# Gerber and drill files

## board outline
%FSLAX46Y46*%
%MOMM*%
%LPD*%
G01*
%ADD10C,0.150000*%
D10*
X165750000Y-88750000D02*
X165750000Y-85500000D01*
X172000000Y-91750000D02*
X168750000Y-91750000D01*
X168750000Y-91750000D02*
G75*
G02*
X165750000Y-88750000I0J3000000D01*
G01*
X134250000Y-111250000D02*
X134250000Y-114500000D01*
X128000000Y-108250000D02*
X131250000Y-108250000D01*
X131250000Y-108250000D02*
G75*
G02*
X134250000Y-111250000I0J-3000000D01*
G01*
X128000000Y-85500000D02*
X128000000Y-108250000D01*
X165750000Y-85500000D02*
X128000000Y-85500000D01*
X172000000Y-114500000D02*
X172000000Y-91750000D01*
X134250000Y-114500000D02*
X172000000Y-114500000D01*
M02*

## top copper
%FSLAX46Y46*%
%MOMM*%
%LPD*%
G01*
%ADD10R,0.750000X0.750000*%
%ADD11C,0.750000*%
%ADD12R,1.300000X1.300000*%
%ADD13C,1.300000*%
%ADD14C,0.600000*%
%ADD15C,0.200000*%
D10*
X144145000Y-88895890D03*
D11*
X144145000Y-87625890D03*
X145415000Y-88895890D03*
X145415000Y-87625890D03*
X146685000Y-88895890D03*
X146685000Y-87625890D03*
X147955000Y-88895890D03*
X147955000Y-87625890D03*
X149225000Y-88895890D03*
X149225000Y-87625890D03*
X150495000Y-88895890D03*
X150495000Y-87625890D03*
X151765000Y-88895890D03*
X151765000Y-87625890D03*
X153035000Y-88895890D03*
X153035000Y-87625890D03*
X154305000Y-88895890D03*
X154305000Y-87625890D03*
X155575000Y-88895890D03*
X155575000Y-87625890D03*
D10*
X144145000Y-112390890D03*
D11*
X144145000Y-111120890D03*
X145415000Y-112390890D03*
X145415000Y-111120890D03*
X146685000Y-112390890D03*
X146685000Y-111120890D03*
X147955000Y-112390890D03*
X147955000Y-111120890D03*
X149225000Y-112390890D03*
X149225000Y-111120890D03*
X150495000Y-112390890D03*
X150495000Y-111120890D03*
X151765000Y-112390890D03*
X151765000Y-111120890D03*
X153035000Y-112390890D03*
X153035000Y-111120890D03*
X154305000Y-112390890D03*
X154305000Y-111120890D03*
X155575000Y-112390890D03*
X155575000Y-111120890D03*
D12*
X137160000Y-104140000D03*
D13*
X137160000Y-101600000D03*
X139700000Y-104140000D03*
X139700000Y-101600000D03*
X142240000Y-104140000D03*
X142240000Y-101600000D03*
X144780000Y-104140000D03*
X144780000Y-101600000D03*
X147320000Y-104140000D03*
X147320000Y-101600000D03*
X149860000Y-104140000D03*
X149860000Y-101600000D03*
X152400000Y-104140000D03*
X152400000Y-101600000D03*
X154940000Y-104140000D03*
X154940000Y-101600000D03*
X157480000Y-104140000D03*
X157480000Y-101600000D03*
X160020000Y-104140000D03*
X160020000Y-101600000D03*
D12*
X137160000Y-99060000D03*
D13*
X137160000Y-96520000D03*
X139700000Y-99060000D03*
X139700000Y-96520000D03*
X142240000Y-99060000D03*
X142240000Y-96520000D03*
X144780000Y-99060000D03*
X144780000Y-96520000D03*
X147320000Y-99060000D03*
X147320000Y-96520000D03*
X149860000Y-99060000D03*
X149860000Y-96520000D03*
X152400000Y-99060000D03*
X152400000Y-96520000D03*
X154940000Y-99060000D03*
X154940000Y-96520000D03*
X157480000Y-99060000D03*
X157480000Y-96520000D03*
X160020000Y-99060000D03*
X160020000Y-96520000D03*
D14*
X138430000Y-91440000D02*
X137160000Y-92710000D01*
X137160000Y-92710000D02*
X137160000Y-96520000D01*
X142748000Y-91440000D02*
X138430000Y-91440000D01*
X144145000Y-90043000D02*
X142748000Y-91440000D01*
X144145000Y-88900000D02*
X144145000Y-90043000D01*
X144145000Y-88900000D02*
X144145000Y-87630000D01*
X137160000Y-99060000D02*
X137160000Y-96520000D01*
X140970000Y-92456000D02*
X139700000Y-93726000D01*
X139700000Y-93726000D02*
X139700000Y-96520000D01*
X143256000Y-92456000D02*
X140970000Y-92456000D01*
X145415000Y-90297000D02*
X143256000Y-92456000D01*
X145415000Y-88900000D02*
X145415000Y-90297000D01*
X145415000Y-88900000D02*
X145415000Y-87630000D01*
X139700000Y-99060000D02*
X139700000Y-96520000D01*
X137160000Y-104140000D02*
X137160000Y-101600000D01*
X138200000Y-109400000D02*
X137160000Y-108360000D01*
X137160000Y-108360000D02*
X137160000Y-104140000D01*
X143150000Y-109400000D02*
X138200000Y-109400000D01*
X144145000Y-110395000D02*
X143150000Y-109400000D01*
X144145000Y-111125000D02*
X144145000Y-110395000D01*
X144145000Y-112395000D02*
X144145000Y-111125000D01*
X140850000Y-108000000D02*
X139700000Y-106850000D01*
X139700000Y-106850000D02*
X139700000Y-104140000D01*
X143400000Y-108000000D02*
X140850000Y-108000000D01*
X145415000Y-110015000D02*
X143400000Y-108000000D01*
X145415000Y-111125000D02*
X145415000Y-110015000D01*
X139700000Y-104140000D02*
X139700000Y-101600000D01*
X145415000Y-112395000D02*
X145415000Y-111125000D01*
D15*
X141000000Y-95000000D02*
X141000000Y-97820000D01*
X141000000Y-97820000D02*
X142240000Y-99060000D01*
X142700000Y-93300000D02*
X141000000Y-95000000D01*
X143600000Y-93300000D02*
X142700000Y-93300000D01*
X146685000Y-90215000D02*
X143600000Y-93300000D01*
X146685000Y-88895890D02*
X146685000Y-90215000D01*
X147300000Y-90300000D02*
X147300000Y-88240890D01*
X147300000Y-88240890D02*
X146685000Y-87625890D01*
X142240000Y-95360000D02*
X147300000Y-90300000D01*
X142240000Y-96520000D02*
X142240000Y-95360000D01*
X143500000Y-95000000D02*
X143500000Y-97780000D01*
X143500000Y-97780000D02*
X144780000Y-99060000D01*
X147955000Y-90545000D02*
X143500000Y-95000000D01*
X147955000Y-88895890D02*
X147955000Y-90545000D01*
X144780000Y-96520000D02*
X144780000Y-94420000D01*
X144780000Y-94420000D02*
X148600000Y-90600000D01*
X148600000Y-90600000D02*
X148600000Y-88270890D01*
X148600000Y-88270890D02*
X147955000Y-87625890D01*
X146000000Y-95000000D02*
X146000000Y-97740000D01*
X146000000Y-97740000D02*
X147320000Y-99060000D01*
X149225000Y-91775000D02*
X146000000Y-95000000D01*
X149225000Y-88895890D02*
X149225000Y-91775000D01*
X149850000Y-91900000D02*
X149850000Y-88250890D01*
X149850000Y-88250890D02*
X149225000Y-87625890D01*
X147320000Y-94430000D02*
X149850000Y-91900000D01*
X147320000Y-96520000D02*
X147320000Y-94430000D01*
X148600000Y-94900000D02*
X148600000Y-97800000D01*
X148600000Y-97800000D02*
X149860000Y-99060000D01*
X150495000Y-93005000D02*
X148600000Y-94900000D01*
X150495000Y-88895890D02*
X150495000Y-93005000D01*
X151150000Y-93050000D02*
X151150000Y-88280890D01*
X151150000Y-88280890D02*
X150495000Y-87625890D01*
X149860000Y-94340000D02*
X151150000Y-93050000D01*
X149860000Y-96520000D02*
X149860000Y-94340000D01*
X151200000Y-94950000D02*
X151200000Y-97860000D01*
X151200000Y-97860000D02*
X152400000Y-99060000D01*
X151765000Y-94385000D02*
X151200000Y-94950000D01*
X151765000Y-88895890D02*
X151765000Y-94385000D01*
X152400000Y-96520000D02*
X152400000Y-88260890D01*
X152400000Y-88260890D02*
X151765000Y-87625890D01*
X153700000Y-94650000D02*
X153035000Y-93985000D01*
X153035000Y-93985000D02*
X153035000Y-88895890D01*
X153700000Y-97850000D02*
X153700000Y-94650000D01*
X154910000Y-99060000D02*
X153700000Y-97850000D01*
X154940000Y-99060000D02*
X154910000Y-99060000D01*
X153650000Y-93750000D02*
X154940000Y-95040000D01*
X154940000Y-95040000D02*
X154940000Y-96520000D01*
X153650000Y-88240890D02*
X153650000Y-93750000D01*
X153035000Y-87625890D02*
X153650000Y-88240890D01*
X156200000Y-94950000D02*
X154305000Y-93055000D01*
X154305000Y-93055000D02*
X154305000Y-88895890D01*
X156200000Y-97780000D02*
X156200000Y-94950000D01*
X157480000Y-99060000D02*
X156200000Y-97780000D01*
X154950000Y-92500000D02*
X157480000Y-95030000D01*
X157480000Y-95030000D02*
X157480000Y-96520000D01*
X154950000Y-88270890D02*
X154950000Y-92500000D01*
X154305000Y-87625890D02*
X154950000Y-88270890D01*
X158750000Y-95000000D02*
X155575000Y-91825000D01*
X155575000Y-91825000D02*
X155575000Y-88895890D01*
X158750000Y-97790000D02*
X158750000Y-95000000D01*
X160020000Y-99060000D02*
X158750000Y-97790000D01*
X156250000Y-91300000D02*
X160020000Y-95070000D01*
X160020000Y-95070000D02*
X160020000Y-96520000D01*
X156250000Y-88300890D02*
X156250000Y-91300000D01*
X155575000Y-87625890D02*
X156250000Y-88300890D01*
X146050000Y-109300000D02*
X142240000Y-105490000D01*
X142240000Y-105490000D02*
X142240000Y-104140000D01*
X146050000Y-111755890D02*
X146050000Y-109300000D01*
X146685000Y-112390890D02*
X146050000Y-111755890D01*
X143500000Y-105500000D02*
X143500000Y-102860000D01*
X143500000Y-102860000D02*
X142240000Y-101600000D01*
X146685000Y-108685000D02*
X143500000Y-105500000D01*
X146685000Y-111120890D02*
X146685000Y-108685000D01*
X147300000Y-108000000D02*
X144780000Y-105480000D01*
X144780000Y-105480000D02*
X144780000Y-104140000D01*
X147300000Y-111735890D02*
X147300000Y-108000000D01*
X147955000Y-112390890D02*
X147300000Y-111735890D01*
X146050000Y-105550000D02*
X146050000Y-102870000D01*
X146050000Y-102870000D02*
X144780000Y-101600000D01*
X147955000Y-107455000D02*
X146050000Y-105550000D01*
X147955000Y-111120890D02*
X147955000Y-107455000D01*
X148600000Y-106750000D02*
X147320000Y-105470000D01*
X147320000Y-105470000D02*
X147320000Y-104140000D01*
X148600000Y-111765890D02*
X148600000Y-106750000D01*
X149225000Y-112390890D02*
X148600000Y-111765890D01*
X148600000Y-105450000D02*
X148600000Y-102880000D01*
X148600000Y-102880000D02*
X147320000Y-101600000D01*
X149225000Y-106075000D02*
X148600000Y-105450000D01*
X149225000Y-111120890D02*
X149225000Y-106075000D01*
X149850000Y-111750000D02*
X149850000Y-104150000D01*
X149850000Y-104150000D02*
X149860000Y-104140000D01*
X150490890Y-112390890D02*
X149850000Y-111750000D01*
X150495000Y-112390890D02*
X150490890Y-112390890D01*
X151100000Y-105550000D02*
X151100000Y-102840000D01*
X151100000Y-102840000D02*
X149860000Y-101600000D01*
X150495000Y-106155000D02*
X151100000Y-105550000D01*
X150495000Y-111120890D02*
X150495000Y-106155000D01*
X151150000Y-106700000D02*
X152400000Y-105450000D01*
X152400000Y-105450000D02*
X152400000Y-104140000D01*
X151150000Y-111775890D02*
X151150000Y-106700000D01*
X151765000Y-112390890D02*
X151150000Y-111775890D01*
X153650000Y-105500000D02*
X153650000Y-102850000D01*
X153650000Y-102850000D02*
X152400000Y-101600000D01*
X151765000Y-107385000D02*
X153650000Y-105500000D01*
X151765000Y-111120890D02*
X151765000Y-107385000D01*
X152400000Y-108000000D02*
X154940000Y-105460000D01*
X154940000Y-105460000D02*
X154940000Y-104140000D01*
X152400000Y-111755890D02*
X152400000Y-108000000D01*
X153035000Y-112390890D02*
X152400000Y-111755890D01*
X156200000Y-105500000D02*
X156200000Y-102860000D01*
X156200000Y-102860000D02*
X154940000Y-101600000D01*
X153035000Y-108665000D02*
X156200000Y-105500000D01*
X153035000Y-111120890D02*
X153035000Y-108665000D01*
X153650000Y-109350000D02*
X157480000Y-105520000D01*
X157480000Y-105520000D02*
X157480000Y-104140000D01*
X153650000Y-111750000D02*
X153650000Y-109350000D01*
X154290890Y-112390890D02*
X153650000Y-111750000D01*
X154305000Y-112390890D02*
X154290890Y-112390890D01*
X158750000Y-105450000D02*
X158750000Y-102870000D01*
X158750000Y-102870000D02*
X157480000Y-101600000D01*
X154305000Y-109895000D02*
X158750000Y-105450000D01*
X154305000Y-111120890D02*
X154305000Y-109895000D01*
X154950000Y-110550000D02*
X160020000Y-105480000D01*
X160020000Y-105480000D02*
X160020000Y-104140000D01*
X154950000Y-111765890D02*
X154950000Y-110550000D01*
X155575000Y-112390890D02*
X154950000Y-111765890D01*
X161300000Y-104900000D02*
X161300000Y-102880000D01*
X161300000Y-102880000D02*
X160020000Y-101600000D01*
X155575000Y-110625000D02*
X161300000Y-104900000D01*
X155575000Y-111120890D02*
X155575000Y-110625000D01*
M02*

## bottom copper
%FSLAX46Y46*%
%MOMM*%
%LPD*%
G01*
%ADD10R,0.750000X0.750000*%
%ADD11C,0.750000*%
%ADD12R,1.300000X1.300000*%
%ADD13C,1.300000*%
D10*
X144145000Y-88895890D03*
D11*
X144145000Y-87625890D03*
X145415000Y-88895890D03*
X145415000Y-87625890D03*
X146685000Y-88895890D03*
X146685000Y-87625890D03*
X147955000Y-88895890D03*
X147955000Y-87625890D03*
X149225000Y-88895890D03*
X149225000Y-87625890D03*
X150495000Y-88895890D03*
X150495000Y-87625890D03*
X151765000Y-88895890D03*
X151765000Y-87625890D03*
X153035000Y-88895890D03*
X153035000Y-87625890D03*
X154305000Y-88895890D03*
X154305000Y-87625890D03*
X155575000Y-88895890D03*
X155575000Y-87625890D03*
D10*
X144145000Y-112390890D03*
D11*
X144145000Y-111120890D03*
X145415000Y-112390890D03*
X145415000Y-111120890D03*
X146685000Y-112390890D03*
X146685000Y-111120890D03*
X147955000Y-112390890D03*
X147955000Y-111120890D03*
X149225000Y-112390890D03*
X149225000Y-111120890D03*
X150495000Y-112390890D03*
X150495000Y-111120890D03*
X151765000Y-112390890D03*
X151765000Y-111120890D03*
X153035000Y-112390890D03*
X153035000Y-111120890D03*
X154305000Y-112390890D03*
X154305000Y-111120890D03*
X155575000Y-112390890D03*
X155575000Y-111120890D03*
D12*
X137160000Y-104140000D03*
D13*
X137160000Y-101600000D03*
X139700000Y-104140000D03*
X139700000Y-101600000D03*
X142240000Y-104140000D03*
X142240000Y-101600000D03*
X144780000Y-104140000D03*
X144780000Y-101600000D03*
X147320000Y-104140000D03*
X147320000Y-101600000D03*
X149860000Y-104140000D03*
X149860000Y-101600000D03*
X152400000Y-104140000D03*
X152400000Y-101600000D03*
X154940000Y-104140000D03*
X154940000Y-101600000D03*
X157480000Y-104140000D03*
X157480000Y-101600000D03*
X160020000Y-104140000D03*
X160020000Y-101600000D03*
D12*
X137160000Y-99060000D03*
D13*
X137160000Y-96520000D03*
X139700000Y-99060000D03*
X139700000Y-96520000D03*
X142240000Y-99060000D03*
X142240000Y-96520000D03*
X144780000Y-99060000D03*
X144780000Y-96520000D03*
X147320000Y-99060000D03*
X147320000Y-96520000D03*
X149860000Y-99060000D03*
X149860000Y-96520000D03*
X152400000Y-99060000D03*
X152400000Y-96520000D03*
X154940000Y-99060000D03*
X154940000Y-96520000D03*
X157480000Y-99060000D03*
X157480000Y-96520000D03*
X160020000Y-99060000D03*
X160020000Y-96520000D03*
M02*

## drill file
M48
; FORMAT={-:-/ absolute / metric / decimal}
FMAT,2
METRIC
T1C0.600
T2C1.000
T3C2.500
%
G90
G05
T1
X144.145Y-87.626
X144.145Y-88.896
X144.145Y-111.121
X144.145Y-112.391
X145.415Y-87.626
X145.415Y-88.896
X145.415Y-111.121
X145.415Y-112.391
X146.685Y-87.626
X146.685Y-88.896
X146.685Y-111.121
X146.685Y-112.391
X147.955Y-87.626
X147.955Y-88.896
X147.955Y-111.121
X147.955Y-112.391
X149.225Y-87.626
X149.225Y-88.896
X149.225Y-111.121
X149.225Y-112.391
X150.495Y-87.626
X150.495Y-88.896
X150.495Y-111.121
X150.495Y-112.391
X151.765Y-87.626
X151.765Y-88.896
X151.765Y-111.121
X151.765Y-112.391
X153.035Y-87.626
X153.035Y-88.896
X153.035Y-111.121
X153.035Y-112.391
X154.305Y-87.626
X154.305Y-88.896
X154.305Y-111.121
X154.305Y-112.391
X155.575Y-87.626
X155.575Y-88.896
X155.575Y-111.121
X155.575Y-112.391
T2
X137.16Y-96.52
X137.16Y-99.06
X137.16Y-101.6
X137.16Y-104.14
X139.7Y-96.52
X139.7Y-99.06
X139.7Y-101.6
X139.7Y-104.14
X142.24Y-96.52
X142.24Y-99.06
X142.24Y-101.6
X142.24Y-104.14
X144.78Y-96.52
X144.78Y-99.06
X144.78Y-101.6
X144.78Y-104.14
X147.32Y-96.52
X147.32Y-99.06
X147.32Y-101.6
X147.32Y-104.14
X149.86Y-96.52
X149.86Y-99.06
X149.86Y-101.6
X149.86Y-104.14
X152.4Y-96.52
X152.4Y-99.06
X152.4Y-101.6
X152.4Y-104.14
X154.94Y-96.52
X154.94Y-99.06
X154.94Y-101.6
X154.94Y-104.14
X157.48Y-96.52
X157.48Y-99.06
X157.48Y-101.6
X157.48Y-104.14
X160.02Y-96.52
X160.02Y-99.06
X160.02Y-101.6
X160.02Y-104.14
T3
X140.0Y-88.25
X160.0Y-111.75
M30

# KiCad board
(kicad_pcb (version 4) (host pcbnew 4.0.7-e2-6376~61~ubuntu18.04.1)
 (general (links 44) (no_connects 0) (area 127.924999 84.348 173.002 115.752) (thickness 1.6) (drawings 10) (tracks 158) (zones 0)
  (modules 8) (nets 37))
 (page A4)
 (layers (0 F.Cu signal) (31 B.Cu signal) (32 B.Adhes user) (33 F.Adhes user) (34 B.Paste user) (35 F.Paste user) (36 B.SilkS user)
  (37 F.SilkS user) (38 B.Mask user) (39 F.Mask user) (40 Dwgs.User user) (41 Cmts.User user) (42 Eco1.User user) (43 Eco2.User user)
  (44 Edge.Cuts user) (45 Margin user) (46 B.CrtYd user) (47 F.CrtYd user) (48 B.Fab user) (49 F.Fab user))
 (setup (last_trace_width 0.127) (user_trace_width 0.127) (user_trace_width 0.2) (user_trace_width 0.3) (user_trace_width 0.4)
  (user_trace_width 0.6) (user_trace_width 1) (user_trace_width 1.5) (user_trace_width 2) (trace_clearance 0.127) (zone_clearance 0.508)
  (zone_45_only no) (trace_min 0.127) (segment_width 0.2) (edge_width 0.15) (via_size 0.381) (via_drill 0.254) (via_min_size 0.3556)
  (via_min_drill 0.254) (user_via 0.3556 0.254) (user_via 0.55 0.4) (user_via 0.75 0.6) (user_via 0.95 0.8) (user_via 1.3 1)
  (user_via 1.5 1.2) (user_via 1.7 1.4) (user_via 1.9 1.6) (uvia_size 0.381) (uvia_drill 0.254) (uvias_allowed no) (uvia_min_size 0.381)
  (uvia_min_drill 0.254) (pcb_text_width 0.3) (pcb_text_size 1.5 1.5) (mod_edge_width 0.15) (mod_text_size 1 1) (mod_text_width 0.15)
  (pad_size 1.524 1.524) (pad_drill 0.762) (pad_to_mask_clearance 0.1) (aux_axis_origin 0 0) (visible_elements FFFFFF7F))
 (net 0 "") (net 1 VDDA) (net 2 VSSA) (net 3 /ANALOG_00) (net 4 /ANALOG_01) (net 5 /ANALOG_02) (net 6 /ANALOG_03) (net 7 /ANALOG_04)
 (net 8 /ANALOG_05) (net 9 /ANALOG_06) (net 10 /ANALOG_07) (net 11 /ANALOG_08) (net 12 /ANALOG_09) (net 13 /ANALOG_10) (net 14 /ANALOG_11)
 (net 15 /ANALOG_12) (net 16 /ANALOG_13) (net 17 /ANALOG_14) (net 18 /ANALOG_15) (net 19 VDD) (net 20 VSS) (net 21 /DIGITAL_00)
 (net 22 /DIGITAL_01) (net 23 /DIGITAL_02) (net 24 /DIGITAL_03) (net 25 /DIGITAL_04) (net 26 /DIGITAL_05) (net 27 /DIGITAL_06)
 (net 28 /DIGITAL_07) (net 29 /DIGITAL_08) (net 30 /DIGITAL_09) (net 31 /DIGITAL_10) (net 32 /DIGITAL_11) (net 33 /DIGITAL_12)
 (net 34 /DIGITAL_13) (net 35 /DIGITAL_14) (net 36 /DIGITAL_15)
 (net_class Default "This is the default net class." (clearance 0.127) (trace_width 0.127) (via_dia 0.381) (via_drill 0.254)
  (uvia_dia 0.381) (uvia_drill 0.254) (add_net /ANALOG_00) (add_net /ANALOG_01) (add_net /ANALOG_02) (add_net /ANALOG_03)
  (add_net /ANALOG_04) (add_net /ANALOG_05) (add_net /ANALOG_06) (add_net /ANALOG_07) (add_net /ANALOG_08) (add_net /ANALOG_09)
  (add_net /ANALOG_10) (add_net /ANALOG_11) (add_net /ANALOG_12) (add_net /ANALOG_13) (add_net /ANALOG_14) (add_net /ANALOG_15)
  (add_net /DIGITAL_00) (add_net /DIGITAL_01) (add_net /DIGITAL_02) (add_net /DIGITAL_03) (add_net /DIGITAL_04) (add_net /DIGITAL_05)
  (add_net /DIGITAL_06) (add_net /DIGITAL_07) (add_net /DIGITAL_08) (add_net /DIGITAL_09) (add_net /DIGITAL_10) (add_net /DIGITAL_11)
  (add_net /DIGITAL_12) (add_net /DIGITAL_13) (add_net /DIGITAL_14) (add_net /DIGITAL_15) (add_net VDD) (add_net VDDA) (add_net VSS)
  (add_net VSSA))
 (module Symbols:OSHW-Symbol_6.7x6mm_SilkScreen (layer F.Cu) (at 165.735 100.33 90)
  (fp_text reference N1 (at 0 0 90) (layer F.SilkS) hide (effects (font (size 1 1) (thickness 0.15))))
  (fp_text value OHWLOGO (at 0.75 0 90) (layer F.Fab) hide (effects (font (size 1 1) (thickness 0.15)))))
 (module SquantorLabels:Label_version (layer F.Cu) (at 170 100 90)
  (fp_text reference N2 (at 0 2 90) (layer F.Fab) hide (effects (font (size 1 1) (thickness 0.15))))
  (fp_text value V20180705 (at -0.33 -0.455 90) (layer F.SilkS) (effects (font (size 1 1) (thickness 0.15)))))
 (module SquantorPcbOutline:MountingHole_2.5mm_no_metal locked (layer F.Cu) (at 140 88.25)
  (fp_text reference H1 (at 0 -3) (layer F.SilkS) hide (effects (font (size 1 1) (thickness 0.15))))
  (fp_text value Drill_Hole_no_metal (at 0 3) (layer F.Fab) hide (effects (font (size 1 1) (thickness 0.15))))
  (pad "" np_thru_hole circle (at 0 0) (size 2.5 2.5) (drill 2.5) (layers *.Cu *.Mask)))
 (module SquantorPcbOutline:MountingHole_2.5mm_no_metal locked (layer F.Cu) (at 160 111.75)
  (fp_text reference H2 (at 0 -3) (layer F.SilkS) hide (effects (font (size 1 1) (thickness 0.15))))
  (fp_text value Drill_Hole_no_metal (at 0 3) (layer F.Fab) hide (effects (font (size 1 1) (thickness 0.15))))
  (pad "" np_thru_hole circle (at 0 0) (size 2.5 2.5) (drill 2.5) (layers *.Cu *.Mask)))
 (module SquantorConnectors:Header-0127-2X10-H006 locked (layer F.Cu) (at 149.86 88.265)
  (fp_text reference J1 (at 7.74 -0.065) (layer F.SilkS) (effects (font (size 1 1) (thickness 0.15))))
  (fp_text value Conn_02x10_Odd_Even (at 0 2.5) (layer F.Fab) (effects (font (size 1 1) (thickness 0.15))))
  (pad 1 thru_hole rect (at -5.715 0.63089) (size 0.75 0.75) (drill 0.6) (layers *.Cu *.Mask) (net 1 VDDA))
  (pad 2 thru_hole circle (at -5.715 -0.63911) (size 0.75 0.75) (drill 0.6) (layers *.Cu *.Mask) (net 1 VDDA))
  (pad 3 thru_hole circle (at -4.445 0.63089) (size 0.75 0.75) (drill 0.6) (layers *.Cu *.Mask) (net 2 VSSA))
  (pad 4 thru_hole circle (at -4.445 -0.63911) (size 0.75 0.75) (drill 0.6) (layers *.Cu *.Mask) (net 2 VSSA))
  (pad 5 thru_hole circle (at -3.175 0.63089) (size 0.75 0.75) (drill 0.6) (layers *.Cu *.Mask) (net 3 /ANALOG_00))
  (pad 6 thru_hole circle (at -3.175 -0.63911) (size 0.75 0.75) (drill 0.6) (layers *.Cu *.Mask) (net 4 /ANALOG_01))
  (pad 7 thru_hole circle (at -1.905 0.63089) (size 0.75 0.75) (drill 0.6) (layers *.Cu *.Mask) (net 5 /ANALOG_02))
  (pad 8 thru_hole circle (at -1.905 -0.63911) (size 0.75 0.75) (drill 0.6) (layers *.Cu *.Mask) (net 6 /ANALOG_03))
  (pad 9 thru_hole circle (at -0.635 0.63089) (size 0.75 0.75) (drill 0.6) (layers *.Cu *.Mask) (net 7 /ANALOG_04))
  (pad 10 thru_hole circle (at -0.635 -0.63911) (size 0.75 0.75) (drill 0.6) (layers *.Cu *.Mask) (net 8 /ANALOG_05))
  (pad 11 thru_hole circle (at 0.635 0.63089) (size 0.75 0.75) (drill 0.6) (layers *.Cu *.Mask) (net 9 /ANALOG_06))
  (pad 12 thru_hole circle (at 0.635 -0.63911) (size 0.75 0.75) (drill 0.6) (layers *.Cu *.Mask) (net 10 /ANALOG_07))
  (pad 13 thru_hole circle (at 1.905 0.63089) (size 0.75 0.75) (drill 0.6) (layers *.Cu *.Mask) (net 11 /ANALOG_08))
  (pad 14 thru_hole circle (at 1.905 -0.63911) (size 0.75 0.75) (drill 0.6) (layers *.Cu *.Mask) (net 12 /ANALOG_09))
  (pad 15 thru_hole circle (at 3.175 0.63089) (size 0.75 0.75) (drill 0.6) (layers *.Cu *.Mask) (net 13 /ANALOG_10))
  (pad 16 thru_hole circle (at 3.175 -0.63911) (size 0.75 0.75) (drill 0.6) (layers *.Cu *.Mask) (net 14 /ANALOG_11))
  (pad 17 thru_hole circle (at 4.445 0.63089) (size 0.75 0.75) (drill 0.6) (layers *.Cu *.Mask) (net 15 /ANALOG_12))
  (pad 18 thru_hole circle (at 4.445 -0.63911) (size 0.75 0.75) (drill 0.6) (layers *.Cu *.Mask) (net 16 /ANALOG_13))
  (pad 19 thru_hole circle (at 5.715 0.63089) (size 0.75 0.75) (drill 0.6) (layers *.Cu *.Mask) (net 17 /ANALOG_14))
  (pad 20 thru_hole circle (at 5.715 -0.63911) (size 0.75 0.75) (drill 0.6) (layers *.Cu *.Mask) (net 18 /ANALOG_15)))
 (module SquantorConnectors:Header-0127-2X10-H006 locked (layer F.Cu) (at 149.86 111.76)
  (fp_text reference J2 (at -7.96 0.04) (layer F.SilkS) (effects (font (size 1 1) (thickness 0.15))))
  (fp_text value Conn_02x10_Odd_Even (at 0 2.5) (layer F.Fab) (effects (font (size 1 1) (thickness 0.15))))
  (pad 1 thru_hole rect (at -5.715 0.63089) (size 0.75 0.75) (drill 0.6) (layers *.Cu *.Mask) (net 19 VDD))
  (pad 2 thru_hole circle (at -5.715 -0.63911) (size 0.75 0.75) (drill 0.6) (layers *.Cu *.Mask) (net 19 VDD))
  (pad 3 thru_hole circle (at -4.445 0.63089) (size 0.75 0.75) (drill 0.6) (layers *.Cu *.Mask) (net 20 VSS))
  (pad 4 thru_hole circle (at -4.445 -0.63911) (size 0.75 0.75) (drill 0.6) (layers *.Cu *.Mask) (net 20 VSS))
  (pad 5 thru_hole circle (at -3.175 0.63089) (size 0.75 0.75) (drill 0.6) (layers *.Cu *.Mask) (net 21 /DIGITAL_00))
  (pad 6 thru_hole circle (at -3.175 -0.63911) (size 0.75 0.75) (drill 0.6) (layers *.Cu *.Mask) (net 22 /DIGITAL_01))
  (pad 7 thru_hole circle (at -1.905 0.63089) (size 0.75 0.75) (drill 0.6) (layers *.Cu *.Mask) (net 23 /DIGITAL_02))
  (pad 8 thru_hole circle (at -1.905 -0.63911) (size 0.75 0.75) (drill 0.6) (layers *.Cu *.Mask) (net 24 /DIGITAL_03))
  (pad 9 thru_hole circle (at -0.635 0.63089) (size 0.75 0.75) (drill 0.6) (layers *.Cu *.Mask) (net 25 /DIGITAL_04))
  (pad 10 thru_hole circle (at -0.635 -0.63911) (size 0.75 0.75) (drill 0.6) (layers *.Cu *.Mask) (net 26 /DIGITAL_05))
  (pad 11 thru_hole circle (at 0.635 0.63089) (size 0.75 0.75) (drill 0.6) (layers *.Cu *.Mask) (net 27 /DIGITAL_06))
  (pad 12 thru_hole circle (at 0.635 -0.63911) (size 0.75 0.75) (drill 0.6) (layers *.Cu *.Mask) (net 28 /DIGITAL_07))
  (pad 13 thru_hole circle (at 1.905 0.63089) (size 0.75 0.75) (drill 0.6) (layers *.Cu *.Mask) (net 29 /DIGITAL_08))
  (pad 14 thru_hole circle (at 1.905 -0.63911) (size 0.75 0.75) (drill 0.6) (layers *.Cu *.Mask) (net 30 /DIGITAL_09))
  (pad 15 thru_hole circle (at 3.175 0.63089) (size 0.75 0.75) (drill 0.6) (layers *.Cu *.Mask) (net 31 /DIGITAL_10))
  (pad 16 thru_hole circle (at 3.175 -0.63911) (size 0.75 0.75) (drill 0.6) (layers *.Cu *.Mask) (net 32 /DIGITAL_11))
  (pad 17 thru_hole circle (at 4.445 0.63089) (size 0.75 0.75) (drill 0.6) (layers *.Cu *.Mask) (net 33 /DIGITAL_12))
  (pad 18 thru_hole circle (at 4.445 -0.63911) (size 0.75 0.75) (drill 0.6) (layers *.Cu *.Mask) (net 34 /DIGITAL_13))
  (pad 19 thru_hole circle (at 5.715 0.63089) (size 0.75 0.75) (drill 0.6) (layers *.Cu *.Mask) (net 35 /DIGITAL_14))
  (pad 20 thru_hole circle (at 5.715 -0.63911) (size 0.75 0.75) (drill 0.6) (layers *.Cu *.Mask) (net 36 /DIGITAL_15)))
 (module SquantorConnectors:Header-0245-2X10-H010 (layer F.Cu) (at 148.59 102.87)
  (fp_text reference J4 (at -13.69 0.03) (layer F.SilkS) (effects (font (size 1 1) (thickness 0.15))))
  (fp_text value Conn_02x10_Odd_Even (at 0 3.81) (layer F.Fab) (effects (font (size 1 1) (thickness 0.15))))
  (pad 1 thru_hole rect (at -11.43 1.27) (size 1.3 1.3) (drill 1) (layers *.Cu *.Mask) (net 19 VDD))
  (pad 2 thru_hole circle (at -11.43 -1.27) (size 1.3 1.3) (drill 1) (layers *.Cu *.Mask) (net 19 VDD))
  (pad 3 thru_hole circle (at -8.89 1.27) (size 1.3 1.3) (drill 1) (layers *.Cu *.Mask) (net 20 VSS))
  (pad 4 thru_hole circle (at -8.89 -1.27) (size 1.3 1.3) (drill 1) (layers *.Cu *.Mask) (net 20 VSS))
  (pad 5 thru_hole circle (at -6.35 1.27) (size 1.3 1.3) (drill 1) (layers *.Cu *.Mask) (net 21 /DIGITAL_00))
  (pad 6 thru_hole circle (at -6.35 -1.27) (size 1.3 1.3) (drill 1) (layers *.Cu *.Mask) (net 22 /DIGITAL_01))
  (pad 7 thru_hole circle (at -3.81 1.27) (size 1.3 1.3) (drill 1) (layers *.Cu *.Mask) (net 23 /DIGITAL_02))
  (pad 8 thru_hole circle (at -3.81 -1.27) (size 1.3 1.3) (drill 1) (layers *.Cu *.Mask) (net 24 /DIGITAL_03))
  (pad 9 thru_hole circle (at -1.27 1.27) (size 1.3 1.3) (drill 1) (layers *.Cu *.Mask) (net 25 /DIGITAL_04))
  (pad 10 thru_hole circle (at -1.27 -1.27) (size 1.3 1.3) (drill 1) (layers *.Cu *.Mask) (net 26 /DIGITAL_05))
  (pad 11 thru_hole circle (at 1.27 1.27) (size 1.3 1.3) (drill 1) (layers *.Cu *.Mask) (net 27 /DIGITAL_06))
  (pad 12 thru_hole circle (at 1.27 -1.27) (size 1.3 1.3) (drill 1) (layers *.Cu *.Mask) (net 28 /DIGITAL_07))
  (pad 13 thru_hole circle (at 3.81 1.27) (size 1.3 1.3) (drill 1) (layers *.Cu *.Mask) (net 29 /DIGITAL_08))
  (pad 14 thru_hole circle (at 3.81 -1.27) (size 1.3 1.3) (drill 1) (layers *.Cu *.Mask) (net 30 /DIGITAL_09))
  (pad 15 thru_hole circle (at 6.35 1.27) (size 1.3 1.3) (drill 1) (layers *.Cu *.Mask) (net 31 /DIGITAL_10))
  (pad 16 thru_hole circle (at 6.35 -1.27) (size 1.3 1.3) (drill 1) (layers *.Cu *.Mask) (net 32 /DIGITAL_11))
  (pad 17 thru_hole circle (at 8.89 1.27) (size 1.3 1.3) (drill 1) (layers *.Cu *.Mask) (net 33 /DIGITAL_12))
  (pad 18 thru_hole circle (at 8.89 -1.27) (size 1.3 1.3) (drill 1) (layers *.Cu *.Mask) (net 34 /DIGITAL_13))
  (pad 19 thru_hole circle (at 11.43 1.27) (size 1.3 1.3) (drill 1) (layers *.Cu *.Mask) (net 35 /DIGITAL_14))
  (pad 20 thru_hole circle (at 11.43 -1.27) (size 1.3 1.3) (drill 1) (layers *.Cu *.Mask) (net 36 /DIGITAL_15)))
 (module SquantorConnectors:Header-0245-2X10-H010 (layer F.Cu) (at 148.59 97.79)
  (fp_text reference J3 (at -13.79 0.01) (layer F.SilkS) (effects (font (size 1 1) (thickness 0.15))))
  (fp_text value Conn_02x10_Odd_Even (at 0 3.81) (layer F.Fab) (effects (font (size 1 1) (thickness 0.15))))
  (pad 1 thru_hole rect (at -11.43 1.27) (size 1.3 1.3) (drill 1) (layers *.Cu *.Mask) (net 1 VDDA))
  (pad 2 thru_hole circle (at -11.43 -1.27) (size 1.3 1.3) (drill 1) (layers *.Cu *.Mask) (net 1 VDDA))
  (pad 3 thru_hole circle (at -8.89 1.27) (size 1.3 1.3) (drill 1) (layers *.Cu *.Mask) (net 2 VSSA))
  (pad 4 thru_hole circle (at -8.89 -1.27) (size 1.3 1.3) (drill 1) (layers *.Cu *.Mask) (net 2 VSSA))
  (pad 5 thru_hole circle (at -6.35 1.27) (size 1.3 1.3) (drill 1) (layers *.Cu *.Mask) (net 3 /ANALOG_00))
  (pad 6 thru_hole circle (at -6.35 -1.27) (size 1.3 1.3) (drill 1) (layers *.Cu *.Mask) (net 4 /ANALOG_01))
  (pad 7 thru_hole circle (at -3.81 1.27) (size 1.3 1.3) (drill 1) (layers *.Cu *.Mask) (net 5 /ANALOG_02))
  (pad 8 thru_hole circle (at -3.81 -1.27) (size 1.3 1.3) (drill 1) (layers *.Cu *.Mask) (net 6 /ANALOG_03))
  (pad 9 thru_hole circle (at -1.27 1.27) (size 1.3 1.3) (drill 1) (layers *.Cu *.Mask) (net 7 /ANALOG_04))
  (pad 10 thru_hole circle (at -1.27 -1.27) (size 1.3 1.3) (drill 1) (layers *.Cu *.Mask) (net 8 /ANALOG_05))
  (pad 11 thru_hole circle (at 1.27 1.27) (size 1.3 1.3) (drill 1) (layers *.Cu *.Mask) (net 9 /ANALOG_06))
  (pad 12 thru_hole circle (at 1.27 -1.27) (size 1.3 1.3) (drill 1) (layers *.Cu *.Mask) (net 10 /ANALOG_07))
  (pad 13 thru_hole circle (at 3.81 1.27) (size 1.3 1.3) (drill 1) (layers *.Cu *.Mask) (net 11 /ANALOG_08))
  (pad 14 thru_hole circle (at 3.81 -1.27) (size 1.3 1.3) (drill 1) (layers *.Cu *.Mask) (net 12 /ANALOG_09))
  (pad 15 thru_hole circle (at 6.35 1.27) (size 1.3 1.3) (drill 1) (layers *.Cu *.Mask) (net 13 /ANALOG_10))
  (pad 16 thru_hole circle (at 6.35 -1.27) (size 1.3 1.3) (drill 1) (layers *.Cu *.Mask) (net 14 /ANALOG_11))
  (pad 17 thru_hole circle (at 8.89 1.27) (size 1.3 1.3) (drill 1) (layers *.Cu *.Mask) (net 15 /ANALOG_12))
  (pad 18 thru_hole circle (at 8.89 -1.27) (size 1.3 1.3) (drill 1) (layers *.Cu *.Mask) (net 16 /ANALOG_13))
  (pad 19 thru_hole circle (at 11.43 1.27) (size 1.3 1.3) (drill 1) (layers *.Cu *.Mask) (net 17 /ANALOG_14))
  (pad 20 thru_hole circle (at 11.43 -1.27) (size 1.3 1.3) (drill 1) (layers *.Cu *.Mask) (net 18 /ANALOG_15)))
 (gr_line (start 165.75 88.75) (end 165.75 85.5) (layer Edge.Cuts) (width 0.15))
 (gr_line (start 172 91.75) (end 168.75 91.75) (layer Edge.Cuts) (width 0.15))
 (gr_arc (start 168.75 88.75) (end 168.75 91.75) (angle 90) (layer Edge.Cuts) (width 0.15))
 (gr_line (start 134.25 111.25) (end 134.25 114.5) (layer Edge.Cuts) (width 0.15))
 (gr_line (start 128 108.25) (end 131.25 108.25) (layer Edge.Cuts) (width 0.15))
 (gr_arc (start 131.25 111.25) (end 131.25 108.25) (angle 90) (layer Edge.Cuts) (width 0.15))
 (gr_line (start 128 85.5) (end 128 108.25) (layer Edge.Cuts) (width 0.15))
 (gr_line (start 165.75 85.5) (end 128 85.5) (layer Edge.Cuts) (width 0.15))
 (gr_line (start 172 114.5) (end 172 91.75) (layer Edge.Cuts) (width 0.15))
 (gr_line (start 134.25 114.5) (end 172 114.5) (layer Edge.Cuts) (width 0.15))
 (segment (start 138.43 91.44) (end 137.16 92.71) (width 0.6) (layer F.Cu) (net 1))
 (segment (start 137.16 92.71) (end 137.16 96.52) (width 0.6) (layer F.Cu) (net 1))
 (segment (start 142.748 91.44) (end 138.43 91.44) (width 0.6) (layer F.Cu) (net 1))
 (segment (start 144.145 90.043) (end 142.748 91.44) (width 0.6) (layer F.Cu) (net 1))
 (segment (start 144.145 88.9) (end 144.145 90.043) (width 0.6) (layer F.Cu) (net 1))
 (segment (start 144.145 88.9) (end 144.145 87.63) (width 0.6) (layer F.Cu) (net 1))
 (segment (start 137.16 99.06) (end 137.16 96.52) (width 0.6) (layer F.Cu) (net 1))
 (segment (start 140.97 92.456) (end 139.7 93.726) (width 0.6) (layer F.Cu) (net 2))
 (segment (start 139.7 93.726) (end 139.7 96.52) (width 0.6) (layer F.Cu) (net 2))
 (segment (start 143.256 92.456) (end 140.97 92.456) (width 0.6) (layer F.Cu) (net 2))
 (segment (start 145.415 90.297) (end 143.256 92.456) (width 0.6) (layer F.Cu) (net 2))
 (segment (start 145.415 88.9) (end 145.415 90.297) (width 0.6) (layer F.Cu) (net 2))
 (segment (start 145.415 88.9) (end 145.415 87.63) (width 0.6) (layer F.Cu) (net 2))
 (segment (start 139.7 99.06) (end 139.7 96.52) (width 0.6) (layer F.Cu) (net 2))
 (segment (start 137.16 104.14) (end 137.16 101.6) (width 0.6) (layer F.Cu) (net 19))
 (segment (start 138.2 109.4) (end 137.16 108.36) (width 0.6) (layer F.Cu) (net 19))
 (segment (start 137.16 108.36) (end 137.16 104.14) (width 0.6) (layer F.Cu) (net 19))
 (segment (start 143.15 109.4) (end 138.2 109.4) (width 0.6) (layer F.Cu) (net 19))
 (segment (start 144.145 110.395) (end 143.15 109.4) (width 0.6) (layer F.Cu) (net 19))
 (segment (start 144.145 111.125) (end 144.145 110.395) (width 0.6) (layer F.Cu) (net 19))
 (segment (start 144.145 112.395) (end 144.145 111.125) (width 0.6) (layer F.Cu) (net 19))
 (segment (start 140.85 108) (end 139.7 106.85) (width 0.6) (layer F.Cu) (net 20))
 (segment (start 139.7 106.85) (end 139.7 104.14) (width 0.6) (layer F.Cu) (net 20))
 (segment (start 143.4 108) (end 140.85 108) (width 0.6) (layer F.Cu) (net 20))
 (segment (start 145.415 110.015) (end 143.4 108) (width 0.6) (layer F.Cu) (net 20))
 (segment (start 145.415 111.125) (end 145.415 110.015) (width 0.6) (layer F.Cu) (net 20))
 (segment (start 139.7 104.14) (end 139.7 101.6) (width 0.6) (layer F.Cu) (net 20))
 (segment (start 145.415 112.395) (end 145.415 111.125) (width 0.6) (layer F.Cu) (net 20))
 (segment (start 141 95) (end 141 97.82) (width 0.2) (layer F.Cu) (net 3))
 (segment (start 141 97.82) (end 142.24 99.06) (width 0.2) (layer F.Cu) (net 3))
 (segment (start 142.7 93.3) (end 141 95) (width 0.2) (layer F.Cu) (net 3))
 (segment (start 143.6 93.3) (end 142.7 93.3) (width 0.2) (layer F.Cu) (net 3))
 (segment (start 146.685 90.215) (end 143.6 93.3) (width 0.2) (layer F.Cu) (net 3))
 (segment (start 146.685 88.89589) (end 146.685 90.215) (width 0.2) (layer F.Cu) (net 3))
 (segment (start 147.3 90.3) (end 147.3 88.24089) (width 0.2) (layer F.Cu) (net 4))
 (segment (start 147.3 88.24089) (end 146.685 87.62589) (width 0.2) (layer F.Cu) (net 4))
 (segment (start 142.24 95.36) (end 147.3 90.3) (width 0.2) (layer F.Cu) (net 4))
 (segment (start 142.24 96.52) (end 142.24 95.36) (width 0.2) (layer F.Cu) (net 4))
 (segment (start 143.5 95) (end 143.5 97.78) (width 0.2) (layer F.Cu) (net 5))
 (segment (start 143.5 97.78) (end 144.78 99.06) (width 0.2) (layer F.Cu) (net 5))
 (segment (start 147.955 90.545) (end 143.5 95) (width 0.2) (layer F.Cu) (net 5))
 (segment (start 147.955 88.89589) (end 147.955 90.545) (width 0.2) (layer F.Cu) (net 5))
 (segment (start 144.78 96.52) (end 144.78 94.42) (width 0.2) (layer F.Cu) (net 6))
 (segment (start 144.78 94.42) (end 148.6 90.6) (width 0.2) (layer F.Cu) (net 6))
 (segment (start 148.6 90.6) (end 148.6 88.27089) (width 0.2) (layer F.Cu) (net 6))
 (segment (start 148.6 88.27089) (end 147.955 87.62589) (width 0.2) (layer F.Cu) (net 6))
 (segment (start 146 95) (end 146 97.74) (width 0.2) (layer F.Cu) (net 7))
 (segment (start 146 97.74) (end 147.32 99.06) (width 0.2) (layer F.Cu) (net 7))
 (segment (start 149.225 91.775) (end 146 95) (width 0.2) (layer F.Cu) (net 7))
 (segment (start 149.225 88.89589) (end 149.225 91.775) (width 0.2) (layer F.Cu) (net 7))
 (segment (start 149.85 91.9) (end 149.85 88.25089) (width 0.2) (layer F.Cu) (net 8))
 (segment (start 149.85 88.25089) (end 149.225 87.62589) (width 0.2) (layer F.Cu) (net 8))
 (segment (start 147.32 94.43) (end 149.85 91.9) (width 0.2) (layer F.Cu) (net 8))
 (segment (start 147.32 96.52) (end 147.32 94.43) (width 0.2) (layer F.Cu) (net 8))
 (segment (start 148.6 94.9) (end 148.6 97.8) (width 0.2) (layer F.Cu) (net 9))
 (segment (start 148.6 97.8) (end 149.86 99.06) (width 0.2) (layer F.Cu) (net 9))
 (segment (start 150.495 93.005) (end 148.6 94.9) (width 0.2) (layer F.Cu) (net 9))
 (segment (start 150.495 88.89589) (end 150.495 93.005) (width 0.2) (layer F.Cu) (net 9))
 (segment (start 151.15 93.05) (end 151.15 88.28089) (width 0.2) (layer F.Cu) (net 10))
 (segment (start 151.15 88.28089) (end 150.495 87.62589) (width 0.2) (layer F.Cu) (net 10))
 (segment (start 149.86 94.34) (end 151.15 93.05) (width 0.2) (layer F.Cu) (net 10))
 (segment (start 149.86 96.52) (end 149.86 94.34) (width 0.2) (layer F.Cu) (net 10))
 (segment (start 151.2 94.95) (end 151.2 97.86) (width 0.2) (layer F.Cu) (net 11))
 (segment (start 151.2 97.86) (end 152.4 99.06) (width 0.2) (layer F.Cu) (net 11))
 (segment (start 151.765 94.385) (end 151.2 94.95) (width 0.2) (layer F.Cu) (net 11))
 (segment (start 151.765 88.89589) (end 151.765 94.385) (width 0.2) (layer F.Cu) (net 11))
 (segment (start 152.4 96.52) (end 152.4 88.26089) (width 0.2) (layer F.Cu) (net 12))
 (segment (start 152.4 88.26089) (end 151.765 87.62589) (width 0.2) (layer F.Cu) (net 12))
 (segment (start 153.7 94.65) (end 153.035 93.985) (width 0.2) (layer F.Cu) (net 13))
 (segment (start 153.035 93.985) (end 153.035 88.89589) (width 0.2) (layer F.Cu) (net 13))
 (segment (start 153.7 97.85) (end 153.7 94.65) (width 0.2) (layer F.Cu) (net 13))
 (segment (start 154.91 99.06) (end 153.7 97.85) (width 0.2) (layer F.Cu) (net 13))
 (segment (start 154.94 99.06) (end 154.91 99.06) (width 0.2) (layer F.Cu) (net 13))
 (segment (start 153.65 93.75) (end 154.94 95.04) (width 0.2) (layer F.Cu) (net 14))
 (segment (start 154.94 95.04) (end 154.94 96.52) (width 0.2) (layer F.Cu) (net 14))
 (segment (start 153.65 88.24089) (end 153.65 93.75) (width 0.2) (layer F.Cu) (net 14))
 (segment (start 153.035 87.62589) (end 153.65 88.24089) (width 0.2) (layer F.Cu) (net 14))
 (segment (start 156.2 94.95) (end 154.305 93.055) (width 0.2) (layer F.Cu) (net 15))
 (segment (start 154.305 93.055) (end 154.305 88.89589) (width 0.2) (layer F.Cu) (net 15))
 (segment (start 156.2 97.78) (end 156.2 94.95) (width 0.2) (layer F.Cu) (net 15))
 (segment (start 157.48 99.06) (end 156.2 97.78) (width 0.2) (layer F.Cu) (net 15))
 (segment (start 154.95 92.5) (end 157.48 95.03) (width 0.2) (layer F.Cu) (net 16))
 (segment (start 157.48 95.03) (end 157.48 96.52) (width 0.2) (layer F.Cu) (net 16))
 (segment (start 154.95 88.27089) (end 154.95 92.5) (width 0.2) (layer F.Cu) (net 16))
 (segment (start 154.305 87.62589) (end 154.95 88.27089) (width 0.2) (layer F.Cu) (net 16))
 (segment (start 158.75 95) (end 155.575 91.825) (width 0.2) (layer F.Cu) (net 17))
 (segment (start 155.575 91.825) (end 155.575 88.89589) (width 0.2) (layer F.Cu) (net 17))
 (segment (start 158.75 97.79) (end 158.75 95) (width 0.2) (layer F.Cu) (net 17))
 (segment (start 160.02 99.06) (end 158.75 97.79) (width 0.2) (layer F.Cu) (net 17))
 (segment (start 156.25 91.3) (end 160.02 95.07) (width 0.2) (layer F.Cu) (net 18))
 (segment (start 160.02 95.07) (end 160.02 96.52) (width 0.2) (layer F.Cu) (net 18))
 (segment (start 156.25 88.30089) (end 156.25 91.3) (width 0.2) (layer F.Cu) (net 18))
 (segment (start 155.575 87.62589) (end 156.25 88.30089) (width 0.2) (layer F.Cu) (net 18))
 (segment (start 146.05 109.3) (end 142.24 105.49) (width 0.2) (layer F.Cu) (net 21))
 (segment (start 142.24 105.49) (end 142.24 104.14) (width 0.2) (layer F.Cu) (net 21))
 (segment (start 146.05 111.75589) (end 146.05 109.3) (width 0.2) (layer F.Cu) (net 21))
 (segment (start 146.685 112.39089) (end 146.05 111.75589) (width 0.2) (layer F.Cu) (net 21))
 (segment (start 143.5 105.5) (end 143.5 102.86) (width 0.2) (layer F.Cu) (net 22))
 (segment (start 143.5 102.86) (end 142.24 101.6) (width 0.2) (layer F.Cu) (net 22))
 (segment (start 146.685 108.685) (end 143.5 105.5) (width 0.2) (layer F.Cu) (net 22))
 (segment (start 146.685 111.12089) (end 146.685 108.685) (width 0.2) (layer F.Cu) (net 22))
 (segment (start 147.3 108) (end 144.78 105.48) (width 0.2) (layer F.Cu) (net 23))
 (segment (start 144.78 105.48) (end 144.78 104.14) (width 0.2) (layer F.Cu) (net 23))
 (segment (start 147.3 111.73589) (end 147.3 108) (width 0.2) (layer F.Cu) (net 23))
 (segment (start 147.955 112.39089) (end 147.3 111.73589) (width 0.2) (layer F.Cu) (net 23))
 (segment (start 146.05 105.55) (end 146.05 102.87) (width 0.2) (layer F.Cu) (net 24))
 (segment (start 146.05 102.87) (end 144.78 101.6) (width 0.2) (layer F.Cu) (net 24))
 (segment (start 147.955 107.455) (end 146.05 105.55) (width 0.2) (layer F.Cu) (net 24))
 (segment (start 147.955 111.12089) (end 147.955 107.455) (width 0.2) (layer F.Cu) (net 24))
 (segment (start 148.6 106.75) (end 147.32 105.47) (width 0.2) (layer F.Cu) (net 25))
 (segment (start 147.32 105.47) (end 147.32 104.14) (width 0.2) (layer F.Cu) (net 25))
 (segment (start 148.6 111.76589) (end 148.6 106.75) (width 0.2) (layer F.Cu) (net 25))
 (segment (start 149.225 112.39089) (end 148.6 111.76589) (width 0.2) (layer F.Cu) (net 25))
 (segment (start 148.6 105.45) (end 148.6 102.88) (width 0.2) (layer F.Cu) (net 26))
 (segment (start 148.6 102.88) (end 147.32 101.6) (width 0.2) (layer F.Cu) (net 26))
 (segment (start 149.225 106.075) (end 148.6 105.45) (width 0.2) (layer F.Cu) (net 26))
 (segment (start 149.225 111.12089) (end 149.225 106.075) (width 0.2) (layer F.Cu) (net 26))
 (segment (start 149.85 111.75) (end 149.85 104.15) (width 0.2) (layer F.Cu) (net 27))
 (segment (start 149.85 104.15) (end 149.86 104.14) (width 0.2) (layer F.Cu) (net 27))
 (segment (start 150.49089 112.39089) (end 149.85 111.75) (width 0.2) (layer F.Cu) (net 27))
 (segment (start 150.495 112.39089) (end 150.49089 112.39089) (width 0.2) (layer F.Cu) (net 27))
 (segment (start 151.1 105.55) (end 151.1 102.84) (width 0.2) (layer F.Cu) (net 28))
 (segment (start 151.1 102.84) (end 149.86 101.6) (width 0.2) (layer F.Cu) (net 28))
 (segment (start 150.495 106.155) (end 151.1 105.55) (width 0.2) (layer F.Cu) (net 28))
 (segment (start 150.495 111.12089) (end 150.495 106.155) (width 0.2) (layer F.Cu) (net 28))
 (segment (start 151.15 106.7) (end 152.4 105.45) (width 0.2) (layer F.Cu) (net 29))
 (segment (start 152.4 105.45) (end 152.4 104.14) (width 0.2) (layer F.Cu) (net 29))
 (segment (start 151.15 111.77589) (end 151.15 106.7) (width 0.2) (layer F.Cu) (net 29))
 (segment (start 151.765 112.39089) (end 151.15 111.77589) (width 0.2) (layer F.Cu) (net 29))
 (segment (start 153.65 105.5) (end 153.65 102.85) (width 0.2) (layer F.Cu) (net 30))
 (segment (start 153.65 102.85) (end 152.4 101.6) (width 0.2) (layer F.Cu) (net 30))
 (segment (start 151.765 107.385) (end 153.65 105.5) (width 0.2) (layer F.Cu) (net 30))
 (segment (start 151.765 111.12089) (end 151.765 107.385) (width 0.2) (layer F.Cu) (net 30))
 (segment (start 152.4 108) (end 154.94 105.46) (width 0.2) (layer F.Cu) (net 31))
 (segment (start 154.94 105.46) (end 154.94 104.14) (width 0.2) (layer F.Cu) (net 31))
 (segment (start 152.4 111.75589) (end 152.4 108) (width 0.2) (layer F.Cu) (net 31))
 (segment (start 153.035 112.39089) (end 152.4 111.75589) (width 0.2) (layer F.Cu) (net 31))
 (segment (start 156.2 105.5) (end 156.2 102.86) (width 0.2) (layer F.Cu) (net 32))
 (segment (start 156.2 102.86) (end 154.94 101.6) (width 0.2) (layer F.Cu) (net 32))
 (segment (start 153.035 108.665) (end 156.2 105.5) (width 0.2) (layer F.Cu) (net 32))
 (segment (start 153.035 111.12089) (end 153.035 108.665) (width 0.2) (layer F.Cu) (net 32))
 (segment (start 153.65 109.35) (end 157.48 105.52) (width 0.2) (layer F.Cu) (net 33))
 (segment (start 157.48 105.52) (end 157.48 104.14) (width 0.2) (layer F.Cu) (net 33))
 (segment (start 153.65 111.75) (end 153.65 109.35) (width 0.2) (layer F.Cu) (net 33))
 (segment (start 154.29089 112.39089) (end 153.65 111.75) (width 0.2) (layer F.Cu) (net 33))
 (segment (start 154.305 112.39089) (end 154.29089 112.39089) (width 0.2) (layer F.Cu) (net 33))
 (segment (start 158.75 105.45) (end 158.75 102.87) (width 0.2) (layer F.Cu) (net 34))
 (segment (start 158.75 102.87) (end 157.48 101.6) (width 0.2) (layer F.Cu) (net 34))
 (segment (start 154.305 109.895) (end 158.75 105.45) (width 0.2) (layer F.Cu) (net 34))
 (segment (start 154.305 111.12089) (end 154.305 109.895) (width 0.2) (layer F.Cu) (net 34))
 (segment (start 154.95 110.55) (end 160.02 105.48) (width 0.2) (layer F.Cu) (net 35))
 (segment (start 160.02 105.48) (end 160.02 104.14) (width 0.2) (layer F.Cu) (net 35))
 (segment (start 154.95 111.76589) (end 154.95 110.55) (width 0.2) (layer F.Cu) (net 35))
 (segment (start 155.575 112.39089) (end 154.95 111.76589) (width 0.2) (layer F.Cu) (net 35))
 (segment (start 161.3 104.9) (end 161.3 102.88) (width 0.2) (layer F.Cu) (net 36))
 (segment (start 161.3 102.88) (end 160.02 101.6) (width 0.2) (layer F.Cu) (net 36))
 (segment (start 155.575 110.625) (end 161.3 104.9) (width 0.2) (layer F.Cu) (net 36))
 (segment (start 155.575 111.12089) (end 155.575 110.625) (width 0.2) (layer F.Cu) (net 36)))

